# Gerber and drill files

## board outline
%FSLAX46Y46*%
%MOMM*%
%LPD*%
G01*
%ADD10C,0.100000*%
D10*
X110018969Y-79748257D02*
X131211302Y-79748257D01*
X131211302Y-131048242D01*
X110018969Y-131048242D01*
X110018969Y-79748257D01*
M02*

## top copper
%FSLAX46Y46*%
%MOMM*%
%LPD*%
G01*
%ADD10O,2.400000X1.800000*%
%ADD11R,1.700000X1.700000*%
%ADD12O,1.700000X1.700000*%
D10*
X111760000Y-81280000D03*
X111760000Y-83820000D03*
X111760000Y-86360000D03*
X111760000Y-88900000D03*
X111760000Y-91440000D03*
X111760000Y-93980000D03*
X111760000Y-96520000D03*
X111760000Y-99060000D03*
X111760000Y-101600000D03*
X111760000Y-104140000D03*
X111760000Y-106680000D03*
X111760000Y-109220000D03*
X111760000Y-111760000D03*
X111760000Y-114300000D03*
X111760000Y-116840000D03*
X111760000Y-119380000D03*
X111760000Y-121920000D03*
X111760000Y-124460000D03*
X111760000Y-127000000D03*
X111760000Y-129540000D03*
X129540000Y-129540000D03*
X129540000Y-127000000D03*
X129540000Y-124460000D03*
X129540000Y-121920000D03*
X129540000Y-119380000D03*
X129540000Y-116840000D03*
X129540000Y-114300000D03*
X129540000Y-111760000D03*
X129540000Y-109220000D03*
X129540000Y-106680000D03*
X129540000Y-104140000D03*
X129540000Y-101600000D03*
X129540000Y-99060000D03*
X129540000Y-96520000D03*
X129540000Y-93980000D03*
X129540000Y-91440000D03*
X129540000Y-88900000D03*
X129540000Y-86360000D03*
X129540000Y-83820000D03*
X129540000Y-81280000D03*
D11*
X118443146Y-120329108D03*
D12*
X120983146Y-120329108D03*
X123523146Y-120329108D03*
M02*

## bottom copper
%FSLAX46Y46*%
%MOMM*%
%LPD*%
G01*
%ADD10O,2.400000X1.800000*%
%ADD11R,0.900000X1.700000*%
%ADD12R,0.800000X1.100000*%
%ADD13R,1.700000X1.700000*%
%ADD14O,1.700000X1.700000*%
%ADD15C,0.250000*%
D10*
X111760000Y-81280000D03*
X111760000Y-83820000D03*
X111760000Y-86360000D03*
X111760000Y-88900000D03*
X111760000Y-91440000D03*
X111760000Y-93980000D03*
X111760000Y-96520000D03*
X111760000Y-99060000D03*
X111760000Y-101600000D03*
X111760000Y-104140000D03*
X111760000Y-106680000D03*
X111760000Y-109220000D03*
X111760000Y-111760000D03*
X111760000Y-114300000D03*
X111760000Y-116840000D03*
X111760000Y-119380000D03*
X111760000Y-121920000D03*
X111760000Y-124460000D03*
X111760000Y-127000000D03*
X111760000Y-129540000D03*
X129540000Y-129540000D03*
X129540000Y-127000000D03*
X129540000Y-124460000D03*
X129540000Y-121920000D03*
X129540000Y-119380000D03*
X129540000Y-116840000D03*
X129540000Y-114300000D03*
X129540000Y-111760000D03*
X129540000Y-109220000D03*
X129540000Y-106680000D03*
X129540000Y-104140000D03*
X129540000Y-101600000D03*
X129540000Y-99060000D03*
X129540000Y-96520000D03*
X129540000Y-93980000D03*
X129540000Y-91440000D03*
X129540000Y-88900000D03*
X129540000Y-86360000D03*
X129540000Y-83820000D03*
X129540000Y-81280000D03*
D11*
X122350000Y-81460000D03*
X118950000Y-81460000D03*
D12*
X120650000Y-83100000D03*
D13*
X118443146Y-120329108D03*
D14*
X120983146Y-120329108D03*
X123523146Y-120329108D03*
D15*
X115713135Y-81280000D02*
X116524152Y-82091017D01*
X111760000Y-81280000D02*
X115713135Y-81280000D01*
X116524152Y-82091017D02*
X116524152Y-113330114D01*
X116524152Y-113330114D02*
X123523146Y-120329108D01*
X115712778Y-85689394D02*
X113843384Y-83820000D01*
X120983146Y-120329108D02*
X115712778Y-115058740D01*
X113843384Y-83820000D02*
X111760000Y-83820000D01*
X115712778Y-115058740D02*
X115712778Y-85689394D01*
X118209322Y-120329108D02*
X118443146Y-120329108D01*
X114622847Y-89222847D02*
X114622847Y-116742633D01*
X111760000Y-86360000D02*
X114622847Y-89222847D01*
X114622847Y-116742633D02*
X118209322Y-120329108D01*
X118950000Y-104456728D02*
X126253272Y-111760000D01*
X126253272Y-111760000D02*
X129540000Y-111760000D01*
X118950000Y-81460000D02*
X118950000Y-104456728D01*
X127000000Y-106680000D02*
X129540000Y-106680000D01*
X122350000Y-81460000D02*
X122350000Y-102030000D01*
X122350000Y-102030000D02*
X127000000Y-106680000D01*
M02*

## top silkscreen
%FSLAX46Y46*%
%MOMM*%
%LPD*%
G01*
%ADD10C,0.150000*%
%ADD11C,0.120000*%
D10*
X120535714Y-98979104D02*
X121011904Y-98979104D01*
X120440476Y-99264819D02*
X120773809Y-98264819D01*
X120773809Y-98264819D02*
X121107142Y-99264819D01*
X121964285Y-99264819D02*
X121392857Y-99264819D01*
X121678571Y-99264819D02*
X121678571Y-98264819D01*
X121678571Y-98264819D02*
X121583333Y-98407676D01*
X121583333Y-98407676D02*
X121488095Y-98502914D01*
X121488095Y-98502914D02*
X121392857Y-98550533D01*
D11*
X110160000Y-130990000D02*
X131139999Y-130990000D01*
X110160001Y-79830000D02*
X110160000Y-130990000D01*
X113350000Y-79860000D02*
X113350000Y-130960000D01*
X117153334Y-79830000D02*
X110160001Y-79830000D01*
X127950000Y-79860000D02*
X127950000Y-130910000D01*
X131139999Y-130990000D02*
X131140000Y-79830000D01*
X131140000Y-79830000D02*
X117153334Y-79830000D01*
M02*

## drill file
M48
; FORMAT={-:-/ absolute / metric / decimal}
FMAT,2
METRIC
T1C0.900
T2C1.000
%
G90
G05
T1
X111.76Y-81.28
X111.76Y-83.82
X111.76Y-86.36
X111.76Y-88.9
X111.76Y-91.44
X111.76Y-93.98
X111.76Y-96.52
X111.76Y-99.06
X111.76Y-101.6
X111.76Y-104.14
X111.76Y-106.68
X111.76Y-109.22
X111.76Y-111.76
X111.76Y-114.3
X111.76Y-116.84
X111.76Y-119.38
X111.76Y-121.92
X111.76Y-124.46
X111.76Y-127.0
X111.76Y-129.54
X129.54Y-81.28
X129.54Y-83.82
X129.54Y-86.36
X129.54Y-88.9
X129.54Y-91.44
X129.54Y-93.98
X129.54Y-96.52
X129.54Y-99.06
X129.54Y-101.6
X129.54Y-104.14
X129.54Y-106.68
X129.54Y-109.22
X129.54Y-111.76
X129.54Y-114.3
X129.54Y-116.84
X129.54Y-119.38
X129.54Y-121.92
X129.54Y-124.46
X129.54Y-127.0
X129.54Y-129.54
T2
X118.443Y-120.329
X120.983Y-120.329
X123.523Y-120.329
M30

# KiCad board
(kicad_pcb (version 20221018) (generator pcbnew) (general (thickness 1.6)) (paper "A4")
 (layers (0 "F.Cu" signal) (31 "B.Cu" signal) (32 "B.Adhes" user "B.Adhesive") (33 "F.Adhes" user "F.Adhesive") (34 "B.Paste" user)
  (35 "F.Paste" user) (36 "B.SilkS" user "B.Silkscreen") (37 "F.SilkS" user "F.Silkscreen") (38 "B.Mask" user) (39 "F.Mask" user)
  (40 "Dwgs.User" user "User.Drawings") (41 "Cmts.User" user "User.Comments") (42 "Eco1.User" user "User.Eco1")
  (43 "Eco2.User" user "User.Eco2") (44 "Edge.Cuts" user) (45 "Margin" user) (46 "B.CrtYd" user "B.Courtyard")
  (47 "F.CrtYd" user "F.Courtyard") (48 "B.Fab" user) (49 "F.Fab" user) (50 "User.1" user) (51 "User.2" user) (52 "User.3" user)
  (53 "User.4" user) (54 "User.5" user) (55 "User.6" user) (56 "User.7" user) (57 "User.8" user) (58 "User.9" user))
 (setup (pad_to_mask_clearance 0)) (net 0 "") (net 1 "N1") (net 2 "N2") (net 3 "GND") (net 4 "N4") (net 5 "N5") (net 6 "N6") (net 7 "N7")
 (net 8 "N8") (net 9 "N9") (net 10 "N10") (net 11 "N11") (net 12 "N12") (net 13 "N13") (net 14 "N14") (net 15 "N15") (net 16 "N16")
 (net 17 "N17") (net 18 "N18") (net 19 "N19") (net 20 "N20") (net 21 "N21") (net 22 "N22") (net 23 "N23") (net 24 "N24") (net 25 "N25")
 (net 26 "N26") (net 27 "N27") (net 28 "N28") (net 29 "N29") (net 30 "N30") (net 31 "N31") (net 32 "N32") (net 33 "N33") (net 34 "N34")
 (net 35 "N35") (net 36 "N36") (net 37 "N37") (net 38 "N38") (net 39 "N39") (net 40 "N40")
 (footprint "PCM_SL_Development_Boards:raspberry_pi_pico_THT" (layer "F.Cu") (at 111.76 81.28)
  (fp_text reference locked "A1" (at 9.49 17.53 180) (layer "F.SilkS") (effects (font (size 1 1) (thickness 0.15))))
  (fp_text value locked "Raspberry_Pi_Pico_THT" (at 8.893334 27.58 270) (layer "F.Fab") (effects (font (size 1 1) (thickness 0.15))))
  (fp_line (start -1.6 49.71) (end 19.379999 49.71) (stroke (width 0.12) (type solid)) (layer "F.SilkS"))
  (fp_line (start -1.599999 -1.45) (end -1.6 49.71) (stroke (width 0.12) (type solid)) (layer "F.SilkS"))
  (fp_line (start 1.59 -1.42) (end 1.59 49.68) (stroke (width 0.12) (type solid)) (layer "F.SilkS"))
  (fp_line (start 5.393334 -1.45) (end -1.599999 -1.45) (stroke (width 0.12) (type solid)) (layer "F.SilkS"))
  (fp_line (start 16.19 -1.42) (end 16.19 49.63) (stroke (width 0.12) (type solid)) (layer "F.SilkS"))
  (fp_line (start 19.379999 49.71) (end 19.38 -1.45) (stroke (width 0.12) (type solid)) (layer "F.SilkS"))
  (fp_line (start 19.38 -1.45) (end 5.393334 -1.45) (stroke (width 0.12) (type solid)) (layer "F.SilkS"))
  (pad "1" thru_hole oval (at 0 0 270) (size 1.8 2.4) (drill 0.9) (layers "*.Cu" "*.Mask") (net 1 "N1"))
  (pad "2" thru_hole oval (at 0 2.54 270) (size 1.8 2.4) (drill 0.9) (layers "*.Cu" "*.Mask") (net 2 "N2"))
  (pad "3" thru_hole oval (at 0 5.08 270) (size 1.8 2.4) (drill 0.9) (layers "*.Cu" "*.Mask") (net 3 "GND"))
  (pad "4" thru_hole oval (at 0 7.62 270) (size 1.8 2.4) (drill 0.9) (layers "*.Cu" "*.Mask") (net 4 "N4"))
  (pad "5" thru_hole oval (at 0 10.16 270) (size 1.8 2.4) (drill 0.9) (layers "*.Cu" "*.Mask") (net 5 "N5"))
  (pad "6" thru_hole oval (at 0 12.7 270) (size 1.8 2.4) (drill 0.9) (layers "*.Cu" "*.Mask") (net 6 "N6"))
  (pad "7" thru_hole oval (at 0 15.24 270) (size 1.8 2.4) (drill 0.9) (layers "*.Cu" "*.Mask") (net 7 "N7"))
  (pad "8" thru_hole oval (at 0 17.78 270) (size 1.8 2.4) (drill 0.9) (layers "*.Cu" "*.Mask") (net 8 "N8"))
  (pad "9" thru_hole oval (at 0 20.32 270) (size 1.8 2.4) (drill 0.9) (layers "*.Cu" "*.Mask") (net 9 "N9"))
  (pad "10" thru_hole oval (at 0 22.86 270) (size 1.8 2.4) (drill 0.9) (layers "*.Cu" "*.Mask") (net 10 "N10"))
  (pad "11" thru_hole oval (at 0 25.4 270) (size 1.8 2.4) (drill 0.9) (layers "*.Cu" "*.Mask") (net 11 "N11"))
  (pad "12" thru_hole oval (at 0 27.94 270) (size 1.8 2.4) (drill 0.9) (layers "*.Cu" "*.Mask") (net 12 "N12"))
  (pad "13" thru_hole oval (at 0 30.48 270) (size 1.8 2.4) (drill 0.9) (layers "*.Cu" "*.Mask") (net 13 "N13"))
  (pad "14" thru_hole oval (at 0 33.02 270) (size 1.8 2.4) (drill 0.9) (layers "*.Cu" "*.Mask") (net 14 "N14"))
  (pad "15" thru_hole oval (at 0 35.56 270) (size 1.8 2.4) (drill 0.9) (layers "*.Cu" "*.Mask") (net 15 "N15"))
  (pad "16" thru_hole oval (at 0 38.1 270) (size 1.8 2.4) (drill 0.9) (layers "*.Cu" "*.Mask") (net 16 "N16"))
  (pad "17" thru_hole oval (at 0 40.64 270) (size 1.8 2.4) (drill 0.9) (layers "*.Cu" "*.Mask") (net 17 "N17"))
  (pad "18" thru_hole oval (at 0 43.18 270) (size 1.8 2.4) (drill 0.9) (layers "*.Cu" "*.Mask") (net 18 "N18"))
  (pad "19" thru_hole oval (at 0 45.72 270) (size 1.8 2.4) (drill 0.9) (layers "*.Cu" "*.Mask") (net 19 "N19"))
  (pad "20" thru_hole oval (at 0 48.26 270) (size 1.8 2.4) (drill 0.9) (layers "*.Cu" "*.Mask") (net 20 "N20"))
  (pad "21" thru_hole oval (at 17.78 48.26 270) (size 1.8 2.4) (drill 0.9) (layers "*.Cu" "*.Mask") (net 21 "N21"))
  (pad "22" thru_hole oval (at 17.78 45.72 270) (size 1.8 2.4) (drill 0.9) (layers "*.Cu" "*.Mask") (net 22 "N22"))
  (pad "23" thru_hole oval (at 17.78 43.18 270) (size 1.8 2.4) (drill 0.9) (layers "*.Cu" "*.Mask") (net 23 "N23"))
  (pad "24" thru_hole oval (at 17.78 40.64 270) (size 1.8 2.4) (drill 0.9) (layers "*.Cu" "*.Mask") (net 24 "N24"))
  (pad "25" thru_hole oval (at 17.78 38.1 270) (size 1.8 2.4) (drill 0.9) (layers "*.Cu" "*.Mask") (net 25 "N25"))
  (pad "26" thru_hole oval (at 17.78 35.56 270) (size 1.8 2.4) (drill 0.9) (layers "*.Cu" "*.Mask") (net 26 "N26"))
  (pad "27" thru_hole oval (at 17.78 33.02 270) (size 1.8 2.4) (drill 0.9) (layers "*.Cu" "*.Mask") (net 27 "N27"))
  (pad "28" thru_hole oval (at 17.78 30.48 270) (size 1.8 2.4) (drill 0.9) (layers "*.Cu" "*.Mask") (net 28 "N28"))
  (pad "29" thru_hole oval (at 17.78 27.94 270) (size 1.8 2.4) (drill 0.9) (layers "*.Cu" "*.Mask") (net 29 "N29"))
  (pad "30" thru_hole oval (at 17.78 25.4 270) (size 1.8 2.4) (drill 0.9) (layers "*.Cu" "*.Mask") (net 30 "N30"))
  (pad "31" thru_hole oval (at 17.78 22.86 270) (size 1.8 2.4) (drill 0.9) (layers "*.Cu" "*.Mask") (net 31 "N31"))
  (pad "32" thru_hole oval (at 17.78 20.32 270) (size 1.8 2.4) (drill 0.9) (layers "*.Cu" "*.Mask") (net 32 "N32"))
  (pad "33" thru_hole oval (at 17.78 17.78 270) (size 1.8 2.4) (drill 0.9) (layers "*.Cu" "*.Mask") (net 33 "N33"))
  (pad "34" thru_hole oval (at 17.78 15.24 270) (size 1.8 2.4) (drill 0.9) (layers "*.Cu" "*.Mask") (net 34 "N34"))
  (pad "35" thru_hole oval (at 17.78 12.7 270) (size 1.8 2.4) (drill 0.9) (layers "*.Cu" "*.Mask") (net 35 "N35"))
  (pad "36" thru_hole oval (at 17.78 10.16 270) (size 1.8 2.4) (drill 0.9) (layers "*.Cu" "*.Mask") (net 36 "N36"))
  (pad "37" thru_hole oval (at 17.78 7.62 270) (size 1.8 2.4) (drill 0.9) (layers "*.Cu" "*.Mask") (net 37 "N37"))
  (pad "38" thru_hole oval (at 17.78 5.08 270) (size 1.8 2.4) (drill 0.9) (layers "*.Cu" "*.Mask") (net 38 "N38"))
  (pad "39" thru_hole oval (at 17.78 2.54 270) (size 1.8 2.4) (drill 0.9) (layers "*.Cu" "*.Mask") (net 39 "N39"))
  (pad "40" thru_hole oval (at 17.78 0 270) (size 1.8 2.4) (drill 0.9) (layers "*.Cu" "*.Mask") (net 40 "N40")))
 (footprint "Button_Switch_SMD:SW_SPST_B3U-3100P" (layer "B.Cu") (at 120.65 82.28 180)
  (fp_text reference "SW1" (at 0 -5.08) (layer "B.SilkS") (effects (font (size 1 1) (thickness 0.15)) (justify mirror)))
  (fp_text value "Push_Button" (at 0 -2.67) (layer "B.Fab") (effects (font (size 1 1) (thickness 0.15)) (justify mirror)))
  (pad "1" smd rect (at -1.7 0.82 180) (size 0.9 1.7) (layers "B.Cu" "B.Paste" "B.Mask") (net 30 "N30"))
  (pad "2" smd rect (at 1.7 0.82 180) (size 0.9 1.7) (layers "B.Cu" "B.Paste" "B.Mask") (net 28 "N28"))
  (pad "3" smd rect (at 0 -0.82 180) (size 0.8 1.1) (layers "B.Cu" "B.Paste" "B.Mask")))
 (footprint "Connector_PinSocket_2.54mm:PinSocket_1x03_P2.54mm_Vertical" (layer "B.Cu") (at 118.443146 120.329108 -90)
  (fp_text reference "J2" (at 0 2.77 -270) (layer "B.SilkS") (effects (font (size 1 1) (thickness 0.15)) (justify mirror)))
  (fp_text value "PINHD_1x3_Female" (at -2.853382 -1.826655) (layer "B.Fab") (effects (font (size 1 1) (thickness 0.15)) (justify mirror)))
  (pad "1" thru_hole rect (at 0 0 270) (size 1.7 1.7) (drill 1) (layers "*.Cu" "*.Mask") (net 3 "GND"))
  (pad "2" thru_hole oval (at 0 -2.54 270) (size 1.7 1.7) (drill 1) (layers "*.Cu" "*.Mask") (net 2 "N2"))
  (pad "3" thru_hole oval (at 0 -5.08 270) (size 1.7 1.7) (drill 1) (layers "*.Cu" "*.Mask") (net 1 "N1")))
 (gr_rect (start 110.018969 79.748257) (end 131.211302 131.048242) (stroke (width 0.1) (type default)) (fill none) (layer "Edge.Cuts"))
 (segment (start 115.713135 81.28) (end 116.524152 82.091017) (width 0.25) (layer "B.Cu") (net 1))
 (segment (start 111.76 81.28) (end 115.713135 81.28) (width 0.25) (layer "B.Cu") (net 1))
 (segment (start 116.524152 82.091017) (end 116.524152 113.330114) (width 0.25) (layer "B.Cu") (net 1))
 (segment (start 116.524152 113.330114) (end 123.523146 120.329108) (width 0.25) (layer "B.Cu") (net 1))
 (segment (start 115.712778 85.689394) (end 113.843384 83.82) (width 0.25) (layer "B.Cu") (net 2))
 (segment (start 120.983146 120.329108) (end 115.712778 115.05874) (width 0.25) (layer "B.Cu") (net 2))
 (segment (start 113.843384 83.82) (end 111.76 83.82) (width 0.25) (layer "B.Cu") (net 2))
 (segment (start 115.712778 115.05874) (end 115.712778 85.689394) (width 0.25) (layer "B.Cu") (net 2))
 (segment (start 118.209322 120.329108) (end 118.443146 120.329108) (width 0.25) (layer "B.Cu") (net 3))
 (segment (start 114.622847 89.222847) (end 114.622847 116.742633) (width 0.25) (layer "B.Cu") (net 3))
 (segment (start 111.76 86.36) (end 114.622847 89.222847) (width 0.25) (layer "B.Cu") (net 3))
 (segment (start 114.622847 116.742633) (end 118.209322 120.329108) (width 0.25) (layer "B.Cu") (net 3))
 (segment (start 118.95 104.456728) (end 126.253272 111.76) (width 0.25) (layer "B.Cu") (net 28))
 (segment (start 126.253272 111.76) (end 129.54 111.76) (width 0.25) (layer "B.Cu") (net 28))
 (segment (start 118.95 81.46) (end 118.95 104.456728) (width 0.25) (layer "B.Cu") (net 28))
 (segment (start 127 106.68) (end 129.54 106.68) (width 0.25) (layer "B.Cu") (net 30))
 (segment (start 122.35 81.46) (end 122.35 102.03) (width 0.25) (layer "B.Cu") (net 30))
 (segment (start 122.35 102.03) (end 127 106.68) (width 0.25) (layer "B.Cu") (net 30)))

